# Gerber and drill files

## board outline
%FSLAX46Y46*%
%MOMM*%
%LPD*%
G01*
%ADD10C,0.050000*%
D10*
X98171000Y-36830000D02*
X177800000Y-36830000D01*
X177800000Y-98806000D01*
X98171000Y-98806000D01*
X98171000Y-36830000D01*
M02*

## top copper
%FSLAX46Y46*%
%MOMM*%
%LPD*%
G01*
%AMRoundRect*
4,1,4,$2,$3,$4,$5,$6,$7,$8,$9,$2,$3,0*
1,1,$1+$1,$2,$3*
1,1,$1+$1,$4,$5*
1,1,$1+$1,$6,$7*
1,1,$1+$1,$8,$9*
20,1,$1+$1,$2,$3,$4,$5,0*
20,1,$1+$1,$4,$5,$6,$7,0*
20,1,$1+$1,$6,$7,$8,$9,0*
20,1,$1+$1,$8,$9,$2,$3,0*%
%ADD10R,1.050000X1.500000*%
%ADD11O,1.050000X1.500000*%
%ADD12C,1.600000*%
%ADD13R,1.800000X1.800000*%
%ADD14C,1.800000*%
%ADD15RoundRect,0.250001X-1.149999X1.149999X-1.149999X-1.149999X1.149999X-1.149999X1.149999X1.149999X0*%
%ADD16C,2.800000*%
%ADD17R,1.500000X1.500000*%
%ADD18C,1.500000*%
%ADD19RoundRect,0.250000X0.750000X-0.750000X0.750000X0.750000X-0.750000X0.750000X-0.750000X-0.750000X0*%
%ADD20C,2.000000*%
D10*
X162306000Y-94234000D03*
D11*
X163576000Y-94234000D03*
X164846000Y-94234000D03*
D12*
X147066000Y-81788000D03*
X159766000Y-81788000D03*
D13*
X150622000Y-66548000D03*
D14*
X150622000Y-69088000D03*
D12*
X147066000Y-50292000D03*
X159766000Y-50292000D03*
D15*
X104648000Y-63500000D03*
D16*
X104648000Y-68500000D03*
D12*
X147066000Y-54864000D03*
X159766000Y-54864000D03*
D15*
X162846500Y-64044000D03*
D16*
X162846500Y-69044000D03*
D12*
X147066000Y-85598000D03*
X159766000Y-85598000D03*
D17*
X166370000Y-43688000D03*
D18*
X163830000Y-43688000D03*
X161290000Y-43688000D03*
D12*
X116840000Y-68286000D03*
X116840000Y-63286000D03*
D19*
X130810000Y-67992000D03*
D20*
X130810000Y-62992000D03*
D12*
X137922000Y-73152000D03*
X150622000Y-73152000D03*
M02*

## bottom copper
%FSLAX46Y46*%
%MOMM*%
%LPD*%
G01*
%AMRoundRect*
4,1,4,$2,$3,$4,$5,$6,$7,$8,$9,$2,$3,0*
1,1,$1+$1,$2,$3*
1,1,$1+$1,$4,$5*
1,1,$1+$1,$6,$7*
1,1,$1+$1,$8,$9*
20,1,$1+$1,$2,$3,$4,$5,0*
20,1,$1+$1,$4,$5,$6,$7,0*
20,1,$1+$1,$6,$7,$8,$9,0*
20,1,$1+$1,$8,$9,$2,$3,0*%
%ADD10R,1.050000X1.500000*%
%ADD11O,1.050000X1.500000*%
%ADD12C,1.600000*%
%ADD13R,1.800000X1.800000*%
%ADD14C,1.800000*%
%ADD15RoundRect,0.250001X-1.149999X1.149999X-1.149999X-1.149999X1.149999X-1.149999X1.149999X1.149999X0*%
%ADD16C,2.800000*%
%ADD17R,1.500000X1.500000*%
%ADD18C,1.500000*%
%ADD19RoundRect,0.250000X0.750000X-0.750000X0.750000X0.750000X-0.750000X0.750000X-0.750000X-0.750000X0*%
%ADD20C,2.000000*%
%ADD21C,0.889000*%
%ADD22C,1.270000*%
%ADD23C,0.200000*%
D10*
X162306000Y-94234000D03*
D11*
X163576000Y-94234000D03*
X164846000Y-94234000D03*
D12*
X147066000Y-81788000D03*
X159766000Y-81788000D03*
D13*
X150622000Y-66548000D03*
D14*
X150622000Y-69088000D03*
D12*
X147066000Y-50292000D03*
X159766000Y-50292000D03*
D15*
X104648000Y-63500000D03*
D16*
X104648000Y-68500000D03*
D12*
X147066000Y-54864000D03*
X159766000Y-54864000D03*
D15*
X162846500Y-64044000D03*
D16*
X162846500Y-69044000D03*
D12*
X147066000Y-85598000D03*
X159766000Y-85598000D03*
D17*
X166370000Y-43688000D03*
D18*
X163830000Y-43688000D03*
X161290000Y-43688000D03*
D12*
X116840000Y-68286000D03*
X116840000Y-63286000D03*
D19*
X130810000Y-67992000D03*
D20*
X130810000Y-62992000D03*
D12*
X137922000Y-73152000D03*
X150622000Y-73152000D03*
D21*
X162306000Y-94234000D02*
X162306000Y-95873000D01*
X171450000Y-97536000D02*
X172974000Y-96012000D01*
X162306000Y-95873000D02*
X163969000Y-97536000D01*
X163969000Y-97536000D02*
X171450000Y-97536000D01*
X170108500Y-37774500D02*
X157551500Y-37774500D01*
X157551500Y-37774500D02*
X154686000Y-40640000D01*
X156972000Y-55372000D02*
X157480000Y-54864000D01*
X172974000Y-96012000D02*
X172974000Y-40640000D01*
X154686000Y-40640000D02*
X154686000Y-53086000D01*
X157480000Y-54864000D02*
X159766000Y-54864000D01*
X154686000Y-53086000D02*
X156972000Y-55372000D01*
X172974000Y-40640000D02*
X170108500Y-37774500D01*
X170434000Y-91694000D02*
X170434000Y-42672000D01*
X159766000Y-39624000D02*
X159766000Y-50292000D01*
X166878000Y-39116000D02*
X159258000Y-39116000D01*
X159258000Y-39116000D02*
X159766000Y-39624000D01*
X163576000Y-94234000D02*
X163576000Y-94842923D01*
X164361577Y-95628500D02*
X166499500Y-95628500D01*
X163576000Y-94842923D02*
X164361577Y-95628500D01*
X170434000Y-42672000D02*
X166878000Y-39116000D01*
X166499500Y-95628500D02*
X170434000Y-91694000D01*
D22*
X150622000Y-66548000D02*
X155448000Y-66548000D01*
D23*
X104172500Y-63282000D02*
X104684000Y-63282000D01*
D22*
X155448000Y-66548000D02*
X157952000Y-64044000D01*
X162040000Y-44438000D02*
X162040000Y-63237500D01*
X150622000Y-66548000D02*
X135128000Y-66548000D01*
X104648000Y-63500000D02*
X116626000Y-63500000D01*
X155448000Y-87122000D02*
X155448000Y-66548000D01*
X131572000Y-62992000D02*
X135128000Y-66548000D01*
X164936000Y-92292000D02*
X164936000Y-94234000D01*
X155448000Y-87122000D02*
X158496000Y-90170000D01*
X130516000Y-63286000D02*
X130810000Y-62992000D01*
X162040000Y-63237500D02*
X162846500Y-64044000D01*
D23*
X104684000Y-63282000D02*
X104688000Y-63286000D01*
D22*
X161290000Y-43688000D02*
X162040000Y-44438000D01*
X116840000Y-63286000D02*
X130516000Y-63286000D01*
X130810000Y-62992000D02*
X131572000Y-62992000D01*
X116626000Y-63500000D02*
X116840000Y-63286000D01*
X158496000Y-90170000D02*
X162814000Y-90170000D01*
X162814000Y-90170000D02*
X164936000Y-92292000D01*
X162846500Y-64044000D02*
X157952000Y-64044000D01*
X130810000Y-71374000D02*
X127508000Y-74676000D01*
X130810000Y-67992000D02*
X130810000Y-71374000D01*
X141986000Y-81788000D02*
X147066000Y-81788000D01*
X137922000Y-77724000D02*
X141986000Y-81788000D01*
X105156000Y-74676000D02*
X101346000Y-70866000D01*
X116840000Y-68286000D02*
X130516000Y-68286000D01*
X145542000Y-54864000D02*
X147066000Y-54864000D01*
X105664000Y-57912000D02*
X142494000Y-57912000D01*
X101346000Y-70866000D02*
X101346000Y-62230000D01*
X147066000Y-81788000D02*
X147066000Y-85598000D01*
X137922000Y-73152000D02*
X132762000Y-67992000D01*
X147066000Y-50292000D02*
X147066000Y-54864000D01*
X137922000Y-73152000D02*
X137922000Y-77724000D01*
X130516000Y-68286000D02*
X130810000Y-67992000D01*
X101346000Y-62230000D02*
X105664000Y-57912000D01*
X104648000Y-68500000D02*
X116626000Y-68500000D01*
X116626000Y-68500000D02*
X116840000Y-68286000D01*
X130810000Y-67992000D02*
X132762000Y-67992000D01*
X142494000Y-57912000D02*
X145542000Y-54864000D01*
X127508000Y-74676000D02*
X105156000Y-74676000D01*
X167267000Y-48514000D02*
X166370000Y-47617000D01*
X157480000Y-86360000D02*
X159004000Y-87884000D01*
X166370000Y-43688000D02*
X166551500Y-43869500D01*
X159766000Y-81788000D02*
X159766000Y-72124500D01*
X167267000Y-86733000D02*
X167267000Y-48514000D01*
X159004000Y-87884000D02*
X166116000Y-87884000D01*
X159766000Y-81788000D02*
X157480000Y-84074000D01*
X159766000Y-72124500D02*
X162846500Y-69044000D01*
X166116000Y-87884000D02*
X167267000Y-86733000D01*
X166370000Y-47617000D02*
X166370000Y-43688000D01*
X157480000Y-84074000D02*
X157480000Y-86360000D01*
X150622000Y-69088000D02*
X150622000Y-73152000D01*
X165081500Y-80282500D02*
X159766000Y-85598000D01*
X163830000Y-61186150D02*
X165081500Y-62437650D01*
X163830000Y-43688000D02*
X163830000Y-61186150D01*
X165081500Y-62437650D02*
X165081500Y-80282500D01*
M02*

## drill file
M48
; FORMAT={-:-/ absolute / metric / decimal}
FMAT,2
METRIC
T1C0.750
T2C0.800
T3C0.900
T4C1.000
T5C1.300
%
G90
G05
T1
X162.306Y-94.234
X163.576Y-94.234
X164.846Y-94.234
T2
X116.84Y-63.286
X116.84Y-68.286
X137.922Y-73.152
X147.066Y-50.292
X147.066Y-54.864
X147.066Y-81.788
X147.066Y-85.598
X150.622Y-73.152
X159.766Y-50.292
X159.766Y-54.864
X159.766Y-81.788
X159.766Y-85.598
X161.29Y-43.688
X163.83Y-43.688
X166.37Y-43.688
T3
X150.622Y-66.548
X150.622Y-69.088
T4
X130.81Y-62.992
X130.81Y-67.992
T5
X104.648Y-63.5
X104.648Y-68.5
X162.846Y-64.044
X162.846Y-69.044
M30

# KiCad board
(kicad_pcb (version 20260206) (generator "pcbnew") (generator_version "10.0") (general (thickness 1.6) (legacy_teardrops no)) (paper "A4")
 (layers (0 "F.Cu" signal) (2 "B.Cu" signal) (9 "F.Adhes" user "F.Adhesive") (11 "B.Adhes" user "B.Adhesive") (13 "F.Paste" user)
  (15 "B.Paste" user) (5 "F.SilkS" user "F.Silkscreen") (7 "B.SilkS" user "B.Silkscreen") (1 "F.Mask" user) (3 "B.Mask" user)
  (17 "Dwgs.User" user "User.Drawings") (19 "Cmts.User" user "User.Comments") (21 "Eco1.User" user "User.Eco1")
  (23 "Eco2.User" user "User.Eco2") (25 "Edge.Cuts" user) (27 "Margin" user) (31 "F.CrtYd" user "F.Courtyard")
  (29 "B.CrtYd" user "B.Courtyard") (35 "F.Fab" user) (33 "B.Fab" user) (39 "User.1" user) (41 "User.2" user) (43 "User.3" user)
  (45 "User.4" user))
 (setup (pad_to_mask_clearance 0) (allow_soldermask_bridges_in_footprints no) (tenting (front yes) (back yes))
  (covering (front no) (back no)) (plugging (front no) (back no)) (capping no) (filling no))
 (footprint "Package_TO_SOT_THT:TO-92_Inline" (layer "F.Cu") (at 162.306 94.234)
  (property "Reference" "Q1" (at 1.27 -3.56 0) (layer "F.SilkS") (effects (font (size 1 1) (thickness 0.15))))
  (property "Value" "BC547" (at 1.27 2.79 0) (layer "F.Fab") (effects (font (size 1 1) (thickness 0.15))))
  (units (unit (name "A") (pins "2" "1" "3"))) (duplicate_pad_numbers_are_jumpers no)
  (pad "1" thru_hole rect (at 0 0) (size 1.05 1.5) (drill 0.75) (layers "*.Cu" "*.Mask") (remove_unused_layers no) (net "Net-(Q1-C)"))
  (pad "2" thru_hole oval (at 1.27 0) (size 1.05 1.5) (drill 0.75) (layers "*.Cu" "*.Mask") (remove_unused_layers no) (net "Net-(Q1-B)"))
  (pad "3" thru_hole oval (at 2.54 0) (size 1.05 1.5) (drill 0.75) (layers "*.Cu" "*.Mask") (remove_unused_layers no) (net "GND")))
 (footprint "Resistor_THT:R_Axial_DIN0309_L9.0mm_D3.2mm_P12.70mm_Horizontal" (layer "F.Cu") (at 147.066 81.788)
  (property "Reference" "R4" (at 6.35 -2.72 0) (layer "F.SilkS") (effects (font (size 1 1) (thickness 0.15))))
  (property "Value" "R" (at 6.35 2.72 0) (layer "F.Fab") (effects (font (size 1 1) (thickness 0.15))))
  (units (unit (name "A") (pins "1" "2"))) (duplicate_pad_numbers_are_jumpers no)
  (pad "1" thru_hole circle (at 0 0) (size 1.6 1.6) (drill 0.8) (layers "*.Cu" "*.Mask") (remove_unused_layers no) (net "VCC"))
  (pad "2" thru_hole circle (at 12.7 0) (size 1.6 1.6) (drill 0.8) (layers "*.Cu" "*.Mask") (remove_unused_layers no) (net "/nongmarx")))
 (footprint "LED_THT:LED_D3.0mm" (layer "F.Cu") (at 150.622 66.548 -90)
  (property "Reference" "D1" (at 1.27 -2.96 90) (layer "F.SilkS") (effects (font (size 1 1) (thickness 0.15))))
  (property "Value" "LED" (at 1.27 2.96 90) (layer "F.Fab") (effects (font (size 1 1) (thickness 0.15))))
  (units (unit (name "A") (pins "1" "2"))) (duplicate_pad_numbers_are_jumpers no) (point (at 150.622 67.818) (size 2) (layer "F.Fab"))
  (pad "1" thru_hole rect (at 0 0 270) (size 1.8 1.8) (drill 0.9) (layers "*.Cu" "*.Mask") (remove_unused_layers no) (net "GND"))
  (pad "2" thru_hole circle (at 2.54 0 270) (size 1.8 1.8) (drill 0.9) (layers "*.Cu" "*.Mask") (remove_unused_layers no) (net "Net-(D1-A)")))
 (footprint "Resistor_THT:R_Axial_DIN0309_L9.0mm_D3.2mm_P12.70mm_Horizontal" (layer "F.Cu") (at 147.066 50.292)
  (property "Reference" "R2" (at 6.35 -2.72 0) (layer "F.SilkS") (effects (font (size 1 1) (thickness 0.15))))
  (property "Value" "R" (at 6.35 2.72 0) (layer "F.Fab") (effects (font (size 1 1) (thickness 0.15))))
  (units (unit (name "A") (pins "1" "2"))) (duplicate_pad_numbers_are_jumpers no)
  (pad "1" thru_hole circle (at 0 0) (size 1.6 1.6) (drill 0.8) (layers "*.Cu" "*.Mask") (remove_unused_layers no) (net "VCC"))
  (pad "2" thru_hole circle (at 12.7 0) (size 1.6 1.6) (drill 0.8) (layers "*.Cu" "*.Mask") (remove_unused_layers no) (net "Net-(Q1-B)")))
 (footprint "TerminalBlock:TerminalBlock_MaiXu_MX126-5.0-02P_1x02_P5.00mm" (layer "F.Cu") (at 104.648 63.5 -90)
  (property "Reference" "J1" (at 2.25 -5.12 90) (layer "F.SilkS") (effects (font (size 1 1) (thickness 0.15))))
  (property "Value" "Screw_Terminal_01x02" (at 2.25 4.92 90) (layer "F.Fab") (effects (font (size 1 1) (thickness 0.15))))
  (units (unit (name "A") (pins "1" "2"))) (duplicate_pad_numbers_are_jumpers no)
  (pad "1" thru_hole roundrect (at 0 0 270) (size 2.8 2.8) (drill 1.3) (layers "*.Cu" "*.Mask") (remove_unused_layers no)
   (roundrect_rratio 0.089286) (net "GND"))
  (pad "2" thru_hole circle (at 5 0 270) (size 2.8 2.8) (drill 1.3) (layers "*.Cu" "*.Mask") (remove_unused_layers no) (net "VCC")))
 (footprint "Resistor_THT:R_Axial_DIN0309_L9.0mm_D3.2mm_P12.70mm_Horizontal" (layer "F.Cu") (at 147.066 54.864)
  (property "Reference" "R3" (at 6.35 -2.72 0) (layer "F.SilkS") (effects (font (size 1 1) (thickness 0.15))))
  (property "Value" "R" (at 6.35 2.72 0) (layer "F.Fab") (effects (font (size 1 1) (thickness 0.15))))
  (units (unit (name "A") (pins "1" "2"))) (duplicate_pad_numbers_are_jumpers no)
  (pad "1" thru_hole circle (at 0 0) (size 1.6 1.6) (drill 0.8) (layers "*.Cu" "*.Mask") (remove_unused_layers no) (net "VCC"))
  (pad "2" thru_hole circle (at 12.7 0) (size 1.6 1.6) (drill 0.8) (layers "*.Cu" "*.Mask") (remove_unused_layers no) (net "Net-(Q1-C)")))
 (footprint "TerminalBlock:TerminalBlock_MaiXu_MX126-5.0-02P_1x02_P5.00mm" (layer "F.Cu") (at 162.8465 64.044 -90)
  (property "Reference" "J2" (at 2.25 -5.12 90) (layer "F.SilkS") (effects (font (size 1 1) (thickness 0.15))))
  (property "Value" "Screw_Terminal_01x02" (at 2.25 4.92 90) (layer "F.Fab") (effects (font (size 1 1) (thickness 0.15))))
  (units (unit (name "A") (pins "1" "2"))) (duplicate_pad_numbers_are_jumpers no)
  (pad "1" thru_hole roundrect (at 0 0 270) (size 2.8 2.8) (drill 1.3) (layers "*.Cu" "*.Mask") (remove_unused_layers no)
   (roundrect_rratio 0.089286) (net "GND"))
  (pad "2" thru_hole circle (at 5 0 270) (size 2.8 2.8) (drill 1.3) (layers "*.Cu" "*.Mask") (remove_unused_layers no) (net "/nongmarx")))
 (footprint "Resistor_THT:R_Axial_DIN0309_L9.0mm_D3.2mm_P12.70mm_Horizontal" (layer "F.Cu") (at 147.066 85.598)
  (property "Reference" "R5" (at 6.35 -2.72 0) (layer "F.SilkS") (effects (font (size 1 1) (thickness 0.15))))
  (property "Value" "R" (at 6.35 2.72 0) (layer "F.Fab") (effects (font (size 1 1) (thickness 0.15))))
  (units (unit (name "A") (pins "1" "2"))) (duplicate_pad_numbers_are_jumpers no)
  (pad "1" thru_hole circle (at 0 0) (size 1.6 1.6) (drill 0.8) (layers "*.Cu" "*.Mask") (remove_unused_layers no) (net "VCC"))
  (pad "2" thru_hole circle (at 12.7 0) (size 1.6 1.6) (drill 0.8) (layers "*.Cu" "*.Mask") (remove_unused_layers no) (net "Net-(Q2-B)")))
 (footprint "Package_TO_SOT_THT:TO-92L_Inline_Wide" (layer "F.Cu") (at 166.37 43.688 180)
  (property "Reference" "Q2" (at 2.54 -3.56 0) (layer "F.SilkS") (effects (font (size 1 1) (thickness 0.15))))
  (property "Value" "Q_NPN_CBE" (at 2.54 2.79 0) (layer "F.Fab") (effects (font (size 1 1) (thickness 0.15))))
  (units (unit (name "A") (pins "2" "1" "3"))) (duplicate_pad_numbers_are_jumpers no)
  (pad "1" thru_hole rect (at 0 0 180) (size 1.5 1.5) (drill 0.8) (layers "*.Cu" "*.Mask") (remove_unused_layers no) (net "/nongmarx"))
  (pad "2" thru_hole circle (at 2.54 0 180) (size 1.5 1.5) (drill 0.8) (layers "*.Cu" "*.Mask") (remove_unused_layers no) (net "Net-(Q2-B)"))
  (pad "3" thru_hole circle (at 5.08 0 180) (size 1.5 1.5) (drill 0.8) (layers "*.Cu" "*.Mask") (remove_unused_layers no) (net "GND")))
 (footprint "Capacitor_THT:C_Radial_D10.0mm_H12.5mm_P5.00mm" (layer "F.Cu") (at 116.84 68.286 90)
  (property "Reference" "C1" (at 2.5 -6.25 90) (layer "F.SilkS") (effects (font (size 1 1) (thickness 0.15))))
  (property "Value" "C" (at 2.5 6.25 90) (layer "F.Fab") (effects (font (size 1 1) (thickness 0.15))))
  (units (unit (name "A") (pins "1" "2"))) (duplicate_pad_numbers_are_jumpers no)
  (pad "1" thru_hole circle (at 0 0 90) (size 1.6 1.6) (drill 0.8) (layers "*.Cu" "*.Mask") (remove_unused_layers no) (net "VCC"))
  (pad "2" thru_hole circle (at 5 0 90) (size 1.6 1.6) (drill 0.8) (layers "*.Cu" "*.Mask") (remove_unused_layers no) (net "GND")))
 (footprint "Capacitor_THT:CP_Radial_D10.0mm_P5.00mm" (layer "F.Cu") (at 130.81 67.992 90)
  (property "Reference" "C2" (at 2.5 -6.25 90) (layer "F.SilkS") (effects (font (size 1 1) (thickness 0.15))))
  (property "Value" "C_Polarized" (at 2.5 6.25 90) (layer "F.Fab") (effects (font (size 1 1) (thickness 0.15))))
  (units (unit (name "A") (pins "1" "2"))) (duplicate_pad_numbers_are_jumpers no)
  (pad "1" thru_hole roundrect (at 0 0 90) (size 2 2) (drill 1) (layers "*.Cu" "*.Mask") (remove_unused_layers no) (roundrect_rratio 0.125)
   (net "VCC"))
  (pad "2" thru_hole circle (at 5 0 90) (size 2 2) (drill 1) (layers "*.Cu" "*.Mask") (remove_unused_layers no) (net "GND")))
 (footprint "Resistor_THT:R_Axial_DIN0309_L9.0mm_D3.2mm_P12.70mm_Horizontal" (layer "F.Cu") (at 137.922 73.152)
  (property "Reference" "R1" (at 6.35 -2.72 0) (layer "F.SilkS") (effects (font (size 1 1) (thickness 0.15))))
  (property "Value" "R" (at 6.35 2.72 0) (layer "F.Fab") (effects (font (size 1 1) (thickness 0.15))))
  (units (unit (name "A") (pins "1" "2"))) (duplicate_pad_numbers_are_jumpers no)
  (pad "1" thru_hole circle (at 0 0) (size 1.6 1.6) (drill 0.8) (layers "*.Cu" "*.Mask") (remove_unused_layers no) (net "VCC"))
  (pad "2" thru_hole circle (at 12.7 0) (size 1.6 1.6) (drill 0.8) (layers "*.Cu" "*.Mask") (remove_unused_layers no) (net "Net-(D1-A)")))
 (gr_rect (start 98.171 36.83) (end 177.8 98.806) (stroke (width 0.05) (type default)) (fill no) (layer "Edge.Cuts"))
 (segment (start 162.306 94.234) (end 162.306 95.873) (width 0.889) (layer "B.Cu") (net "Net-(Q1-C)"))
 (segment (start 171.45 97.536) (end 172.974 96.012) (width 0.889) (layer "B.Cu") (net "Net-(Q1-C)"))
 (segment (start 162.306 95.873) (end 163.969 97.536) (width 0.889) (layer "B.Cu") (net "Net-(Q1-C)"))
 (segment (start 163.969 97.536) (end 171.45 97.536) (width 0.889) (layer "B.Cu") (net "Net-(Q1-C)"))
 (segment (start 170.1085 37.7745) (end 157.5515 37.7745) (width 0.889) (layer "B.Cu") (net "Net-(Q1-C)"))
 (segment (start 157.5515 37.7745) (end 154.686 40.64) (width 0.889) (layer "B.Cu") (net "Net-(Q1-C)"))
 (segment (start 156.972 55.372) (end 157.48 54.864) (width 0.889) (layer "B.Cu") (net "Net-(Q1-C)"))
 (segment (start 172.974 96.012) (end 172.974 40.64) (width 0.889) (layer "B.Cu") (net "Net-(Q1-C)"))
 (segment (start 154.686 40.64) (end 154.686 53.086) (width 0.889) (layer "B.Cu") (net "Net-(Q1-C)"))
 (segment (start 157.48 54.864) (end 159.766 54.864) (width 0.889) (layer "B.Cu") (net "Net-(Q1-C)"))
 (segment (start 154.686 53.086) (end 156.972 55.372) (width 0.889) (layer "B.Cu") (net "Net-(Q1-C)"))
 (segment (start 172.974 40.64) (end 170.1085 37.7745) (width 0.889) (layer "B.Cu") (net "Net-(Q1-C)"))
 (segment (start 170.434 91.694) (end 170.434 42.672) (width 0.889) (layer "B.Cu") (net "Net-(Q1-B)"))
 (segment (start 159.766 39.624) (end 159.766 50.292) (width 0.889) (layer "B.Cu") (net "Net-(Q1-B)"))
 (segment (start 166.878 39.116) (end 159.258 39.116) (width 0.889) (layer "B.Cu") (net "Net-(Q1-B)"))
 (segment (start 159.258 39.116) (end 159.766 39.624) (width 0.889) (layer "B.Cu") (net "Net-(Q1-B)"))
 (segment (start 163.576 94.234) (end 163.576 94.842923) (width 0.889) (layer "B.Cu") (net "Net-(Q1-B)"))
 (segment (start 164.361577 95.6285) (end 166.4995 95.6285) (width 0.889) (layer "B.Cu") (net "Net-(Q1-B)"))
 (segment (start 163.576 94.842923) (end 164.361577 95.6285) (width 0.889) (layer "B.Cu") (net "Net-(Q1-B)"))
 (segment (start 170.434 42.672) (end 166.878 39.116) (width 0.889) (layer "B.Cu") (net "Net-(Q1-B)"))
 (segment (start 166.4995 95.6285) (end 170.434 91.694) (width 0.889) (layer "B.Cu") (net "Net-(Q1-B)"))
 (segment (start 150.622 66.548) (end 155.448 66.548) (width 1.27) (layer "B.Cu") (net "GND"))
 (segment (start 104.1725 63.282) (end 104.684 63.282) (width 0.2) (layer "B.Cu") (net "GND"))
 (segment (start 155.448 66.548) (end 157.952 64.044) (width 1.27) (layer "B.Cu") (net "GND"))
 (segment (start 162.04 44.438) (end 162.04 63.2375) (width 1.27) (layer "B.Cu") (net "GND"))
 (segment (start 150.622 66.548) (end 135.128 66.548) (width 1.27) (layer "B.Cu") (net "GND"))
 (segment (start 104.648 63.5) (end 116.626 63.5) (width 1.27) (layer "B.Cu") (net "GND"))
 (segment (start 155.448 87.122) (end 155.448 66.548) (width 1.27) (layer "B.Cu") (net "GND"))
 (segment (start 131.572 62.992) (end 135.128 66.548) (width 1.27) (layer "B.Cu") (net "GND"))
 (segment (start 164.936 92.292) (end 164.936 94.234) (width 1.27) (layer "B.Cu") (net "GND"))
 (segment (start 155.448 87.122) (end 158.496 90.17) (width 1.27) (layer "B.Cu") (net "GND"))
 (segment (start 130.516 63.286) (end 130.81 62.992) (width 1.27) (layer "B.Cu") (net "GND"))
 (segment (start 162.04 63.2375) (end 162.8465 64.044) (width 1.27) (layer "B.Cu") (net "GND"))
 (segment (start 104.684 63.282) (end 104.688 63.286) (width 0.2) (layer "B.Cu") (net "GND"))
 (segment (start 161.29 43.688) (end 162.04 44.438) (width 1.27) (layer "B.Cu") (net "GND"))
 (segment (start 116.84 63.286) (end 130.516 63.286) (width 1.27) (layer "B.Cu") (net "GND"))
 (segment (start 130.81 62.992) (end 131.572 62.992) (width 1.27) (layer "B.Cu") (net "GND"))
 (segment (start 116.626 63.5) (end 116.84 63.286) (width 1.27) (layer "B.Cu") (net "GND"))
 (segment (start 158.496 90.17) (end 162.814 90.17) (width 1.27) (layer "B.Cu") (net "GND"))
 (segment (start 162.814 90.17) (end 164.936 92.292) (width 1.27) (layer "B.Cu") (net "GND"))
 (segment (start 162.8465 64.044) (end 157.952 64.044) (width 1.27) (layer "B.Cu") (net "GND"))
 (segment (start 130.81 71.374) (end 127.508 74.676) (width 1.27) (layer "B.Cu") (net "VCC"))
 (segment (start 130.81 67.992) (end 130.81 71.374) (width 1.27) (layer "B.Cu") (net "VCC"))
 (segment (start 141.986 81.788) (end 147.066 81.788) (width 1.27) (layer "B.Cu") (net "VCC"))
 (segment (start 137.922 77.724) (end 141.986 81.788) (width 1.27) (layer "B.Cu") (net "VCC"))
 (segment (start 105.156 74.676) (end 101.346 70.866) (width 1.27) (layer "B.Cu") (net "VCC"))
 (segment (start 116.84 68.286) (end 130.516 68.286) (width 1.27) (layer "B.Cu") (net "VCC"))
 (segment (start 145.542 54.864) (end 147.066 54.864) (width 1.27) (layer "B.Cu") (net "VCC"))
 (segment (start 105.664 57.912) (end 142.494 57.912) (width 1.27) (layer "B.Cu") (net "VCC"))
 (segment (start 101.346 70.866) (end 101.346 62.23) (width 1.27) (layer "B.Cu") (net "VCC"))
 (segment (start 147.066 81.788) (end 147.066 85.598) (width 1.27) (layer "B.Cu") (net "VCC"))
 (segment (start 137.922 73.152) (end 132.762 67.992) (width 1.27) (layer "B.Cu") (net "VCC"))
 (segment (start 147.066 50.292) (end 147.066 54.864) (width 1.27) (layer "B.Cu") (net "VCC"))
 (segment (start 137.922 73.152) (end 137.922 77.724) (width 1.27) (layer "B.Cu") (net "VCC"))
 (segment (start 130.516 68.286) (end 130.81 67.992) (width 1.27) (layer "B.Cu") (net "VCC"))
 (segment (start 101.346 62.23) (end 105.664 57.912) (width 1.27) (layer "B.Cu") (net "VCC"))
 (segment (start 104.648 68.5) (end 116.626 68.5) (width 1.27) (layer "B.Cu") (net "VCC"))
 (segment (start 116.626 68.5) (end 116.84 68.286) (width 1.27) (layer "B.Cu") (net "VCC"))
 (segment (start 130.81 67.992) (end 132.762 67.992) (width 1.27) (layer "B.Cu") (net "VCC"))
 (segment (start 142.494 57.912) (end 145.542 54.864) (width 1.27) (layer "B.Cu") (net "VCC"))
 (segment (start 127.508 74.676) (end 105.156 74.676) (width 1.27) (layer "B.Cu") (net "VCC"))
 (segment (start 167.267 48.514) (end 166.37 47.617) (width 1.27) (layer "B.Cu") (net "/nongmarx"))
 (segment (start 157.48 86.36) (end 159.004 87.884) (width 1.27) (layer "B.Cu") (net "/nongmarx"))
 (segment (start 166.37 43.688) (end 166.5515 43.8695) (width 1.27) (layer "B.Cu") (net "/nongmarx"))
 (segment (start 159.766 81.788) (end 159.766 72.1245) (width 1.27) (layer "B.Cu") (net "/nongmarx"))
 (segment (start 167.267 86.733) (end 167.267 48.514) (width 1.27) (layer "B.Cu") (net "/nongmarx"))
 (segment (start 159.004 87.884) (end 166.116 87.884) (width 1.27) (layer "B.Cu") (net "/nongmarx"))
 (segment (start 159.766 81.788) (end 157.48 84.074) (width 1.27) (layer "B.Cu") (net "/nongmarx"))
 (segment (start 159.766 72.1245) (end 162.8465 69.044) (width 1.27) (layer "B.Cu") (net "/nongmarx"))
 (segment (start 166.116 87.884) (end 167.267 86.733) (width 1.27) (layer "B.Cu") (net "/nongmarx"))
 (segment (start 166.37 47.617) (end 166.37 43.688) (width 1.27) (layer "B.Cu") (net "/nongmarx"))
 (segment (start 157.48 84.074) (end 157.48 86.36) (width 1.27) (layer "B.Cu") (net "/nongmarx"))
 (segment (start 150.622 69.088) (end 150.622 73.152) (width 1.27) (layer "B.Cu") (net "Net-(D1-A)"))
 (segment (start 165.0815 80.2825) (end 159.766 85.598) (width 1.27) (layer "B.Cu") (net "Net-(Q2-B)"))
 (segment (start 163.83 61.18615) (end 165.0815 62.43765) (width 1.27) (layer "B.Cu") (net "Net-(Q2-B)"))
 (segment (start 163.83 43.688) (end 163.83 61.18615) (width 1.27) (layer "B.Cu") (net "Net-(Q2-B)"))
 (segment (start 165.0815 62.43765) (end 165.0815 80.2825) (width 1.27) (layer "B.Cu") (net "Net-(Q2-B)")))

